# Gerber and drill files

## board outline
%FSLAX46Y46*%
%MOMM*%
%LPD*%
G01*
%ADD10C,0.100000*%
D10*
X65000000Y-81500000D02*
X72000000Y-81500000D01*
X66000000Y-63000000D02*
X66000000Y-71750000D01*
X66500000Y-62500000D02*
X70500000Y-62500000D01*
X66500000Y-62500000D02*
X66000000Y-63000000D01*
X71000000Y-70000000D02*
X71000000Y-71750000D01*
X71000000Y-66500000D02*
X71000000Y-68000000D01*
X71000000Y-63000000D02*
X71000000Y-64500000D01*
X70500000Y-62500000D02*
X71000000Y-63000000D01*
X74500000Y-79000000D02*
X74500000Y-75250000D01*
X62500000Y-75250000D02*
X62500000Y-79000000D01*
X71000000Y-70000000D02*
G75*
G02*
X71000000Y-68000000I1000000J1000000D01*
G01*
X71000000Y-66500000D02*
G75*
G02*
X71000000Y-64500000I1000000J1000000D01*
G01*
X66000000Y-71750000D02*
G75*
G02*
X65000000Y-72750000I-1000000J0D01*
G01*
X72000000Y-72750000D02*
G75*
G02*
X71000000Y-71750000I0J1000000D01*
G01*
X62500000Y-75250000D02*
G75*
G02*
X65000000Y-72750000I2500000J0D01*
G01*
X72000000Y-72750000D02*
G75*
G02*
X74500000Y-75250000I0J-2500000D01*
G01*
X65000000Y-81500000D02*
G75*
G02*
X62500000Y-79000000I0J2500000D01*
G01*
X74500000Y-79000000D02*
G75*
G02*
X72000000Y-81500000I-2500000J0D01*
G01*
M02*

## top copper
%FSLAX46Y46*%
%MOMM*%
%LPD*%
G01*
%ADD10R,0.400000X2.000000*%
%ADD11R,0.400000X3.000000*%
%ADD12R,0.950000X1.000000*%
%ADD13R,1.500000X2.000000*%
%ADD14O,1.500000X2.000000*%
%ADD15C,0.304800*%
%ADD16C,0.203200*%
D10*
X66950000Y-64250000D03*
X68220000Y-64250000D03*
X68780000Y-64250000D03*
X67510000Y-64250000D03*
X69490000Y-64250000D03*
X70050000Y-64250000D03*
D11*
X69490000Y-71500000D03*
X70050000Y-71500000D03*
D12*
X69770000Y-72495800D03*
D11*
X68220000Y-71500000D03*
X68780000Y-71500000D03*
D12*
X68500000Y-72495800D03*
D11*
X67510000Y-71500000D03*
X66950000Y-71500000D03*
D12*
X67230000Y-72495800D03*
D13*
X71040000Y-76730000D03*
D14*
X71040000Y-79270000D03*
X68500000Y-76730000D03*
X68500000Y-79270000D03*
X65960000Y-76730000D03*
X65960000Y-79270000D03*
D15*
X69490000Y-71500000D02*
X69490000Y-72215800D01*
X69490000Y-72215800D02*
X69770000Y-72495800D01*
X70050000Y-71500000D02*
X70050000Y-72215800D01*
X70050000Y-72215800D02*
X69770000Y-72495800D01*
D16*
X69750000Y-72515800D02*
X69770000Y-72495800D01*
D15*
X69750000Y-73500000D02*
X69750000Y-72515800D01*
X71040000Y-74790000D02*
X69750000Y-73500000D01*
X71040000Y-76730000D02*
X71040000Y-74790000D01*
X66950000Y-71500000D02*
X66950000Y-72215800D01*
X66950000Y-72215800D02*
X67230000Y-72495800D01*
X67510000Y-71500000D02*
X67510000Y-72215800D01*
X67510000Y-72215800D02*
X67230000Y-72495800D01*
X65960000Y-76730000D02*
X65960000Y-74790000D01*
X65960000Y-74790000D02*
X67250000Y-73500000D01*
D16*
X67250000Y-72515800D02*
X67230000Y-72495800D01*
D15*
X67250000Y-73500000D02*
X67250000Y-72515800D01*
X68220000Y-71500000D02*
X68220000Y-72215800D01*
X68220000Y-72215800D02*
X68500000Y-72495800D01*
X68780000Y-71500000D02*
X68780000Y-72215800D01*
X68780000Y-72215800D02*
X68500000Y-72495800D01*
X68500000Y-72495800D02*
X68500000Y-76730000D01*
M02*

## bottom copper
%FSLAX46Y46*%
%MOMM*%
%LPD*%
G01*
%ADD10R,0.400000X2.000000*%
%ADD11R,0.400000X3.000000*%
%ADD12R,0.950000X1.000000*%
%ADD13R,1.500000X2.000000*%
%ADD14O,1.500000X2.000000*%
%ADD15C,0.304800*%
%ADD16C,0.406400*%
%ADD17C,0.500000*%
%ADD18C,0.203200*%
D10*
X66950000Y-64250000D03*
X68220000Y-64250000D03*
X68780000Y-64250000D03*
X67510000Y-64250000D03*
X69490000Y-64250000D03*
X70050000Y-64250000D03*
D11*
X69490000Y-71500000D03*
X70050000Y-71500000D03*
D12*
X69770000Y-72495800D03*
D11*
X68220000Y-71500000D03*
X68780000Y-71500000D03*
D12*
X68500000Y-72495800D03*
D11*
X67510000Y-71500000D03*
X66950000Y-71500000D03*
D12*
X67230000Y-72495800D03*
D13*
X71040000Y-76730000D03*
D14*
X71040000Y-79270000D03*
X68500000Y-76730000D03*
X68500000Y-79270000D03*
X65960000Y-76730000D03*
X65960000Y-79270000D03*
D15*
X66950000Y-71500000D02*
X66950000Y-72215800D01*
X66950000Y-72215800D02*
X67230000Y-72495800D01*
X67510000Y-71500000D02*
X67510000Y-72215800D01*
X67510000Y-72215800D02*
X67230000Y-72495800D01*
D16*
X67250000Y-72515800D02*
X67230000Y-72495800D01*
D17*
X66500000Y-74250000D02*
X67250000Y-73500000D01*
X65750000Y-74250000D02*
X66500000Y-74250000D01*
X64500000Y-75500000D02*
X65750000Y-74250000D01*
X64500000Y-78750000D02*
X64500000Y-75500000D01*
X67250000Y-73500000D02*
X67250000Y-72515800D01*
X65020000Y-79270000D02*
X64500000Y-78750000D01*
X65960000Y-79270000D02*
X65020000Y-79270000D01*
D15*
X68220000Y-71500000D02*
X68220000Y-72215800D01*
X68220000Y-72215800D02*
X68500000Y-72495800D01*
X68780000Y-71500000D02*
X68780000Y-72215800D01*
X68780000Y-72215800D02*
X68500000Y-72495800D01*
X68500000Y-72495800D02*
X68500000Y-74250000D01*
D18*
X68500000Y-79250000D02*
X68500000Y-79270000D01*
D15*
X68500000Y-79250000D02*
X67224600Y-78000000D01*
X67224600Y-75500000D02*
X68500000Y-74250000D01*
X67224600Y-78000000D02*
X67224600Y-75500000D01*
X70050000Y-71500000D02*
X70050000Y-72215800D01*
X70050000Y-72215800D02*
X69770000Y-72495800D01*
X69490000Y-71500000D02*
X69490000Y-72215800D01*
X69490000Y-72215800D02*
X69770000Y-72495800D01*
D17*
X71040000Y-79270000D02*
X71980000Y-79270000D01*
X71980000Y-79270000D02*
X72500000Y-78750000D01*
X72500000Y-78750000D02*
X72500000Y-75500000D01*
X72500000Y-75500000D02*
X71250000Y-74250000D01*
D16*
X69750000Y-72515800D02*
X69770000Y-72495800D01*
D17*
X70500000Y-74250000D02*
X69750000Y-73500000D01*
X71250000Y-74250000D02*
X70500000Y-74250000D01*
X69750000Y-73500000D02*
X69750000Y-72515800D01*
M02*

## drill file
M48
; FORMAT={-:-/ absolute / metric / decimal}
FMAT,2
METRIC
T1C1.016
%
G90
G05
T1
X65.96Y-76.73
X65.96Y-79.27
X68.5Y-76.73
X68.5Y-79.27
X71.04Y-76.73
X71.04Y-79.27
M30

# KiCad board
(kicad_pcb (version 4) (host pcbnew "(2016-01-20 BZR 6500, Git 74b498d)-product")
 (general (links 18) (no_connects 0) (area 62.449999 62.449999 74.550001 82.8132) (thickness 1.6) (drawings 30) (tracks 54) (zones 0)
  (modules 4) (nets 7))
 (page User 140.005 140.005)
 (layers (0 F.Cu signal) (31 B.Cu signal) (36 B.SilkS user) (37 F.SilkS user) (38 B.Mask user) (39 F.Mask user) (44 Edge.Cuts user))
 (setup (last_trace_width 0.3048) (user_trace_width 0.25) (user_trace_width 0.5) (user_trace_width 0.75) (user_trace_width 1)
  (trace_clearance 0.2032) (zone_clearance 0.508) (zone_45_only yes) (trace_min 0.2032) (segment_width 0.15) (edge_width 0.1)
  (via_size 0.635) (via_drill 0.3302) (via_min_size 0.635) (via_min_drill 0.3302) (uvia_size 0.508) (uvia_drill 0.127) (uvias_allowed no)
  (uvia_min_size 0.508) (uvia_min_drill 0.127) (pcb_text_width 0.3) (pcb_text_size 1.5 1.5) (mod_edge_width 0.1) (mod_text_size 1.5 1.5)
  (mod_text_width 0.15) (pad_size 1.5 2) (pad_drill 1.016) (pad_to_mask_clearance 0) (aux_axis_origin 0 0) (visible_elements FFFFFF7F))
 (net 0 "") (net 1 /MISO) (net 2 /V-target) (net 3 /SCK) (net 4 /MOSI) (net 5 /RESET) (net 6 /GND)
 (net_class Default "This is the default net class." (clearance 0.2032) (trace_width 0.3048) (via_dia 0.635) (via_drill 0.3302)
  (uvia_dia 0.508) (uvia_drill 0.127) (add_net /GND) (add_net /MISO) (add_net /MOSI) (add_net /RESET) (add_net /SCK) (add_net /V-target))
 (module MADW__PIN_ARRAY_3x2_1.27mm (layer F.Cu) (at 68.5 68) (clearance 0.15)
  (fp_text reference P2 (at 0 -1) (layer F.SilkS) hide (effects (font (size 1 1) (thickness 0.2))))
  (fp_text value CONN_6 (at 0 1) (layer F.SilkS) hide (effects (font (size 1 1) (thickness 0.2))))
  (pad ~ smd rect (at -1.55 -3.75) (size 0.4 2) (layers F.Cu F.Mask))
  (pad ~ smd rect (at -0.28 -3.75) (size 0.4 2) (layers F.Cu F.Mask))
  (pad ~ smd rect (at 0.28 -3.75) (size 0.4 2) (layers F.Cu F.Mask))
  (pad ~ smd rect (at -0.99 -3.75) (size 0.4 2) (layers F.Cu F.Mask))
  (pad ~ smd rect (at 0.99 -3.75) (size 0.4 2) (layers F.Cu F.Mask))
  (pad ~ smd rect (at 1.55 -3.75) (size 0.4 2) (layers F.Cu F.Mask))
  (pad ~ smd rect (at -1.55 -3.75) (size 0.4 2) (layers B.Cu F.Mask))
  (pad ~ smd rect (at -0.28 -3.75) (size 0.4 2) (layers B.Cu F.Mask))
  (pad ~ smd rect (at 0.28 -3.75) (size 0.4 2) (layers B.Cu F.Mask))
  (pad ~ smd rect (at -0.99 -3.75) (size 0.4 2) (layers B.Cu F.Mask))
  (pad ~ smd rect (at 0.99 -3.75) (size 0.4 2) (layers B.Cu F.Mask))
  (pad ~ smd rect (at 1.55 -3.75) (size 0.4 2) (layers B.Cu F.Mask))
  (pad 1 smd rect (at 0.99 3.5) (size 0.4 3) (layers F.Cu F.Mask) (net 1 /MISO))
  (pad 1 smd rect (at 1.55 3.5) (size 0.4 3) (layers F.Cu F.Mask) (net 1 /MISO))
  (pad 1 smd rect (at 1.27 4.4958) (size 0.95 1) (layers F.Cu F.Mask) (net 1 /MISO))
  (pad 2 smd rect (at 0.99 3.5) (size 0.4 3) (layers B.Cu F.Mask) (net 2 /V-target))
  (pad 2 smd rect (at 1.55 3.5) (size 0.4 3) (layers B.Cu F.Mask) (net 2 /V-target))
  (pad 2 smd rect (at 1.27 4.4958) (size 0.95 1) (layers B.Cu B.Mask) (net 2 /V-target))
  (pad 3 smd rect (at -0.28 3.5) (size 0.4 3) (layers F.Cu F.Mask) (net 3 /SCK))
  (pad 3 smd rect (at 0.28 3.5) (size 0.4 3) (layers F.Cu F.Mask) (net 3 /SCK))
  (pad 3 smd rect (at 0 4.4958) (size 0.95 1) (layers F.Cu F.Mask) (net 3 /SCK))
  (pad 4 smd rect (at -0.28 3.5) (size 0.4 3) (layers B.Cu F.Mask) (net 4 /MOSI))
  (pad 4 smd rect (at 0.28 3.5) (size 0.4 3) (layers B.Cu F.Mask) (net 4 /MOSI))
  (pad 4 smd rect (at 0 4.4958) (size 0.95 1) (layers B.Cu B.Mask) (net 4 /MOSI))
  (pad 5 smd rect (at -0.99 3.5) (size 0.4 3) (layers F.Cu F.Mask) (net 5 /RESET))
  (pad 5 smd rect (at -1.55 3.5) (size 0.4 3) (layers F.Cu F.Mask) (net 5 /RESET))
  (pad 5 smd rect (at -1.27 4.4958) (size 0.95 1) (layers F.Cu F.Mask) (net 5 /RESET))
  (pad 6 smd rect (at -0.99 3.5) (size 0.4 3) (layers B.Cu F.Mask) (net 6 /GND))
  (pad 6 smd rect (at -1.55 3.5) (size 0.4 3) (layers B.Cu F.Mask) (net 6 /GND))
  (pad 6 smd rect (at -1.27 4.4958) (size 0.95 1) (layers B.Cu B.Mask) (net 6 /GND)))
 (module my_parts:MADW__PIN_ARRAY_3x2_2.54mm (layer F.Cu) (at 68.5 78)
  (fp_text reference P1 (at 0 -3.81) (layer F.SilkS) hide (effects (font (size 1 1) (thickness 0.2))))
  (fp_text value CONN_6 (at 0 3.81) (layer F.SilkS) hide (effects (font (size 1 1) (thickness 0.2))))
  (pad 1 thru_hole rect (at 2.54 -1.27) (size 1.5 2) (drill 1.016) (layers *.Cu *.Mask F.SilkS) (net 1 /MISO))
  (pad 2 thru_hole oval (at 2.54 1.27) (size 1.5 2) (drill 1.016) (layers *.Cu *.Mask F.SilkS) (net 2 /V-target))
  (pad 3 thru_hole oval (at 0 -1.27) (size 1.5 2) (drill 1.016) (layers *.Cu *.Mask F.SilkS) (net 3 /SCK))
  (pad 4 thru_hole oval (at 0 1.27) (size 1.5 2) (drill 1.016) (layers *.Cu *.Mask F.SilkS) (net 4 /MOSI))
  (pad 5 thru_hole oval (at -2.54 -1.27) (size 1.5 2) (drill 1.016) (layers *.Cu *.Mask F.SilkS) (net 5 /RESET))
  (pad 6 thru_hole oval (at -2.54 1.27) (size 1.5 2) (drill 1.016) (layers *.Cu *.Mask F.SilkS) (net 6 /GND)))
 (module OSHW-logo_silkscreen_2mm (layer F.Cu) (at 71.95 74.2)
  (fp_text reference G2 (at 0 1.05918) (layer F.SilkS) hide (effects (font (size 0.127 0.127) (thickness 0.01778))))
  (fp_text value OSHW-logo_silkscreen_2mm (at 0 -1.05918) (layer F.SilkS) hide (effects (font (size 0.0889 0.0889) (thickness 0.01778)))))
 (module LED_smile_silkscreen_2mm (layer F.Cu) (at 64.75 74.25)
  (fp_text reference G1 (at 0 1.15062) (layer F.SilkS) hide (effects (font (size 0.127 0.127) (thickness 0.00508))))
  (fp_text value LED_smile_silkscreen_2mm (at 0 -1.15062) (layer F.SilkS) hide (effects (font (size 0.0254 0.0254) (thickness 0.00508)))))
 (gr_line (start 65 81.5) (end 72 81.5) (layer Edge.Cuts) (width 0.1))
 (gr_line (start 66 63) (end 66 71.75) (angle 90) (layer Edge.Cuts) (width 0.1))
 (gr_line (start 66.5 62.5) (end 70.5 62.5) (angle 90) (layer Edge.Cuts) (width 0.1))
 (gr_line (start 66.5 62.5) (end 66 63) (angle 90) (layer Edge.Cuts) (width 0.1))
 (gr_line (start 71 70) (end 71 71.75) (angle 90) (layer Edge.Cuts) (width 0.1))
 (gr_line (start 71 66.5) (end 71 68) (angle 90) (layer Edge.Cuts) (width 0.1))
 (gr_line (start 71 63) (end 71 64.5) (angle 90) (layer Edge.Cuts) (width 0.1))
 (gr_line (start 70.5 62.5) (end 71 63) (angle 90) (layer Edge.Cuts) (width 0.1))
 (gr_line (start 74.5 79) (end 74.5 75.25) (angle 90) (layer Edge.Cuts) (width 0.1))
 (gr_line (start 62.5 75.25) (end 62.5 79) (angle 90) (layer Edge.Cuts) (width 0.1))
 (gr_arc (start 72 69) (end 71 70) (angle 90) (layer Edge.Cuts) (width 0.1))
 (gr_arc (start 72 65.5) (end 71 66.5) (angle 90) (layer Edge.Cuts) (width 0.1))
 (gr_arc (start 65 71.75) (end 66 71.75) (angle 90) (layer Edge.Cuts) (width 0.1))
 (gr_arc (start 72 71.75) (end 72 72.75) (angle 90) (layer Edge.Cuts) (width 0.1))
 (gr_arc (start 65 75.25) (end 62.5 75.25) (angle 90) (layer Edge.Cuts) (width 0.1))
 (gr_arc (start 72 75.25) (end 72 72.75) (angle 90) (layer Edge.Cuts) (width 0.1))
 (gr_arc (start 65 79) (end 65 81.5) (angle 90) (layer Edge.Cuts) (width 0.1))
 (gr_arc (start 72 79) (end 74.5 79) (angle 90) (layer Edge.Cuts) (width 0.1))
 (segment (start 66.95 71.5) (end 66.95 72.2158) (width 0.3048) (layer B.Cu) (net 6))
 (segment (start 66.95 72.2158) (end 67.23 72.4958) (width 0.3048) (layer B.Cu) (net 6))
 (segment (start 67.51 71.5) (end 67.51 72.2158) (width 0.3048) (layer B.Cu) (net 6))
 (segment (start 67.51 72.2158) (end 67.23 72.4958) (width 0.3048) (layer B.Cu) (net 6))
 (segment (start 67.25 72.5158) (end 67.23 72.4958) (width 0.4064) (layer B.Cu) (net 6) (status 30))
 (segment (start 66.5 74.25) (end 67.25 73.5) (width 0.5) (layer B.Cu) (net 6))
 (segment (start 65.75 74.25) (end 66.5 74.25) (width 0.5) (layer B.Cu) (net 6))
 (segment (start 64.5 75.5) (end 65.75 74.25) (width 0.5) (layer B.Cu) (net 6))
 (segment (start 64.5 78.75) (end 64.5 75.5) (width 0.5) (layer B.Cu) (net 6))
 (segment (start 67.25 73.5) (end 67.25 72.5158) (width 0.5) (layer B.Cu) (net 6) (status 20))
 (segment (start 65.02 79.27) (end 64.5 78.75) (width 0.5) (layer B.Cu) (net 6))
 (segment (start 65.96 79.27) (end 65.02 79.27) (width 0.5) (layer B.Cu) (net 6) (status 10))
 (segment (start 69.49 71.5) (end 69.49 72.2158) (width 0.3048) (layer F.Cu) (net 1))
 (segment (start 69.49 72.2158) (end 69.77 72.4958) (width 0.3048) (layer F.Cu) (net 1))
 (segment (start 70.05 71.5) (end 70.05 72.2158) (width 0.3048) (layer F.Cu) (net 1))
 (segment (start 70.05 72.2158) (end 69.77 72.4958) (width 0.3048) (layer F.Cu) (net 1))
 (segment (start 69.75 72.5158) (end 69.77 72.4958) (width 0.2032) (layer F.Cu) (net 1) (status 30))
 (segment (start 69.75 73.5) (end 69.75 72.5158) (width 0.3048) (layer F.Cu) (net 1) (status 20))
 (segment (start 71.04 74.79) (end 69.75 73.5) (width 0.3048) (layer F.Cu) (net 1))
 (segment (start 71.04 76.73) (end 71.04 74.79) (width 0.3048) (layer F.Cu) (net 1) (status 10))
 (segment (start 68.22 71.5) (end 68.22 72.2158) (width 0.3048) (layer B.Cu) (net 4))
 (segment (start 68.22 72.2158) (end 68.5 72.4958) (width 0.3048) (layer B.Cu) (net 4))
 (segment (start 68.78 71.5) (end 68.78 72.2158) (width 0.3048) (layer B.Cu) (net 4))
 (segment (start 68.78 72.2158) (end 68.5 72.4958) (width 0.3048) (layer B.Cu) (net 4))
 (segment (start 68.5 72.4958) (end 68.5 74.25) (width 0.3048) (layer B.Cu) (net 4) (status 10))
 (segment (start 68.5 79.25) (end 68.5 79.27) (width 0.2032) (layer B.Cu) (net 4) (status 30))
 (segment (start 68.5 79.25) (end 67.2246 78) (width 0.3048) (layer B.Cu) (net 4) (status 10))
 (segment (start 67.2246 75.5) (end 68.5 74.25) (width 0.3048) (layer B.Cu) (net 4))
 (segment (start 67.2246 78) (end 67.2246 75.5) (width 0.3048) (layer B.Cu) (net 4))
 (segment (start 66.95 71.5) (end 66.95 72.2158) (width 0.3048) (layer F.Cu) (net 5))
 (segment (start 66.95 72.2158) (end 67.23 72.4958) (width 0.3048) (layer F.Cu) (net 5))
 (segment (start 67.51 71.5) (end 67.51 72.2158) (width 0.3048) (layer F.Cu) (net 5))
 (segment (start 67.51 72.2158) (end 67.23 72.4958) (width 0.3048) (layer F.Cu) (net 5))
 (segment (start 65.96 76.73) (end 65.96 74.79) (width 0.3048) (layer F.Cu) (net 5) (status 10))
 (segment (start 65.96 74.79) (end 67.25 73.5) (width 0.3048) (layer F.Cu) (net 5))
 (segment (start 67.25 72.5158) (end 67.23 72.4958) (width 0.2032) (layer F.Cu) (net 5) (status 30))
 (segment (start 67.25 73.5) (end 67.25 72.5158) (width 0.3048) (layer F.Cu) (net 5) (status 20))
 (segment (start 68.22 71.5) (end 68.22 72.2158) (width 0.3048) (layer F.Cu) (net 3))
 (segment (start 68.22 72.2158) (end 68.5 72.4958) (width 0.3048) (layer F.Cu) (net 3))
 (segment (start 68.78 71.5) (end 68.78 72.2158) (width 0.3048) (layer F.Cu) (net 3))
 (segment (start 68.78 72.2158) (end 68.5 72.4958) (width 0.3048) (layer F.Cu) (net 3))
 (segment (start 68.5 72.4958) (end 68.5 76.73) (width 0.3048) (layer F.Cu) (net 3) (status 30))
 (segment (start 70.05 71.5) (end 70.05 72.2158) (width 0.3048) (layer B.Cu) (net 2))
 (segment (start 70.05 72.2158) (end 69.77 72.4958) (width 0.3048) (layer B.Cu) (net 2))
 (segment (start 69.49 71.5) (end 69.49 72.2158) (width 0.3048) (layer B.Cu) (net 2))
 (segment (start 69.49 72.2158) (end 69.77 72.4958) (width 0.3048) (layer B.Cu) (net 2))
 (segment (start 71.04 79.27) (end 71.98 79.27) (width 0.5) (layer B.Cu) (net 2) (status 10))
 (segment (start 71.98 79.27) (end 72.5 78.75) (width 0.5) (layer B.Cu) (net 2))
 (segment (start 72.5 78.75) (end 72.5 75.5) (width 0.5) (layer B.Cu) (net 2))
 (segment (start 72.5 75.5) (end 71.25 74.25) (width 0.5) (layer B.Cu) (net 2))
 (segment (start 69.75 72.5158) (end 69.77 72.4958) (width 0.4064) (layer B.Cu) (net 2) (status 30))
 (segment (start 70.5 74.25) (end 69.75 73.5) (width 0.5) (layer B.Cu) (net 2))
 (segment (start 71.25 74.25) (end 70.5 74.25) (width 0.5) (layer B.Cu) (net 2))
 (segment (start 69.75 73.5) (end 69.75 72.5158) (width 0.5) (layer B.Cu) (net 2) (status 20)))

